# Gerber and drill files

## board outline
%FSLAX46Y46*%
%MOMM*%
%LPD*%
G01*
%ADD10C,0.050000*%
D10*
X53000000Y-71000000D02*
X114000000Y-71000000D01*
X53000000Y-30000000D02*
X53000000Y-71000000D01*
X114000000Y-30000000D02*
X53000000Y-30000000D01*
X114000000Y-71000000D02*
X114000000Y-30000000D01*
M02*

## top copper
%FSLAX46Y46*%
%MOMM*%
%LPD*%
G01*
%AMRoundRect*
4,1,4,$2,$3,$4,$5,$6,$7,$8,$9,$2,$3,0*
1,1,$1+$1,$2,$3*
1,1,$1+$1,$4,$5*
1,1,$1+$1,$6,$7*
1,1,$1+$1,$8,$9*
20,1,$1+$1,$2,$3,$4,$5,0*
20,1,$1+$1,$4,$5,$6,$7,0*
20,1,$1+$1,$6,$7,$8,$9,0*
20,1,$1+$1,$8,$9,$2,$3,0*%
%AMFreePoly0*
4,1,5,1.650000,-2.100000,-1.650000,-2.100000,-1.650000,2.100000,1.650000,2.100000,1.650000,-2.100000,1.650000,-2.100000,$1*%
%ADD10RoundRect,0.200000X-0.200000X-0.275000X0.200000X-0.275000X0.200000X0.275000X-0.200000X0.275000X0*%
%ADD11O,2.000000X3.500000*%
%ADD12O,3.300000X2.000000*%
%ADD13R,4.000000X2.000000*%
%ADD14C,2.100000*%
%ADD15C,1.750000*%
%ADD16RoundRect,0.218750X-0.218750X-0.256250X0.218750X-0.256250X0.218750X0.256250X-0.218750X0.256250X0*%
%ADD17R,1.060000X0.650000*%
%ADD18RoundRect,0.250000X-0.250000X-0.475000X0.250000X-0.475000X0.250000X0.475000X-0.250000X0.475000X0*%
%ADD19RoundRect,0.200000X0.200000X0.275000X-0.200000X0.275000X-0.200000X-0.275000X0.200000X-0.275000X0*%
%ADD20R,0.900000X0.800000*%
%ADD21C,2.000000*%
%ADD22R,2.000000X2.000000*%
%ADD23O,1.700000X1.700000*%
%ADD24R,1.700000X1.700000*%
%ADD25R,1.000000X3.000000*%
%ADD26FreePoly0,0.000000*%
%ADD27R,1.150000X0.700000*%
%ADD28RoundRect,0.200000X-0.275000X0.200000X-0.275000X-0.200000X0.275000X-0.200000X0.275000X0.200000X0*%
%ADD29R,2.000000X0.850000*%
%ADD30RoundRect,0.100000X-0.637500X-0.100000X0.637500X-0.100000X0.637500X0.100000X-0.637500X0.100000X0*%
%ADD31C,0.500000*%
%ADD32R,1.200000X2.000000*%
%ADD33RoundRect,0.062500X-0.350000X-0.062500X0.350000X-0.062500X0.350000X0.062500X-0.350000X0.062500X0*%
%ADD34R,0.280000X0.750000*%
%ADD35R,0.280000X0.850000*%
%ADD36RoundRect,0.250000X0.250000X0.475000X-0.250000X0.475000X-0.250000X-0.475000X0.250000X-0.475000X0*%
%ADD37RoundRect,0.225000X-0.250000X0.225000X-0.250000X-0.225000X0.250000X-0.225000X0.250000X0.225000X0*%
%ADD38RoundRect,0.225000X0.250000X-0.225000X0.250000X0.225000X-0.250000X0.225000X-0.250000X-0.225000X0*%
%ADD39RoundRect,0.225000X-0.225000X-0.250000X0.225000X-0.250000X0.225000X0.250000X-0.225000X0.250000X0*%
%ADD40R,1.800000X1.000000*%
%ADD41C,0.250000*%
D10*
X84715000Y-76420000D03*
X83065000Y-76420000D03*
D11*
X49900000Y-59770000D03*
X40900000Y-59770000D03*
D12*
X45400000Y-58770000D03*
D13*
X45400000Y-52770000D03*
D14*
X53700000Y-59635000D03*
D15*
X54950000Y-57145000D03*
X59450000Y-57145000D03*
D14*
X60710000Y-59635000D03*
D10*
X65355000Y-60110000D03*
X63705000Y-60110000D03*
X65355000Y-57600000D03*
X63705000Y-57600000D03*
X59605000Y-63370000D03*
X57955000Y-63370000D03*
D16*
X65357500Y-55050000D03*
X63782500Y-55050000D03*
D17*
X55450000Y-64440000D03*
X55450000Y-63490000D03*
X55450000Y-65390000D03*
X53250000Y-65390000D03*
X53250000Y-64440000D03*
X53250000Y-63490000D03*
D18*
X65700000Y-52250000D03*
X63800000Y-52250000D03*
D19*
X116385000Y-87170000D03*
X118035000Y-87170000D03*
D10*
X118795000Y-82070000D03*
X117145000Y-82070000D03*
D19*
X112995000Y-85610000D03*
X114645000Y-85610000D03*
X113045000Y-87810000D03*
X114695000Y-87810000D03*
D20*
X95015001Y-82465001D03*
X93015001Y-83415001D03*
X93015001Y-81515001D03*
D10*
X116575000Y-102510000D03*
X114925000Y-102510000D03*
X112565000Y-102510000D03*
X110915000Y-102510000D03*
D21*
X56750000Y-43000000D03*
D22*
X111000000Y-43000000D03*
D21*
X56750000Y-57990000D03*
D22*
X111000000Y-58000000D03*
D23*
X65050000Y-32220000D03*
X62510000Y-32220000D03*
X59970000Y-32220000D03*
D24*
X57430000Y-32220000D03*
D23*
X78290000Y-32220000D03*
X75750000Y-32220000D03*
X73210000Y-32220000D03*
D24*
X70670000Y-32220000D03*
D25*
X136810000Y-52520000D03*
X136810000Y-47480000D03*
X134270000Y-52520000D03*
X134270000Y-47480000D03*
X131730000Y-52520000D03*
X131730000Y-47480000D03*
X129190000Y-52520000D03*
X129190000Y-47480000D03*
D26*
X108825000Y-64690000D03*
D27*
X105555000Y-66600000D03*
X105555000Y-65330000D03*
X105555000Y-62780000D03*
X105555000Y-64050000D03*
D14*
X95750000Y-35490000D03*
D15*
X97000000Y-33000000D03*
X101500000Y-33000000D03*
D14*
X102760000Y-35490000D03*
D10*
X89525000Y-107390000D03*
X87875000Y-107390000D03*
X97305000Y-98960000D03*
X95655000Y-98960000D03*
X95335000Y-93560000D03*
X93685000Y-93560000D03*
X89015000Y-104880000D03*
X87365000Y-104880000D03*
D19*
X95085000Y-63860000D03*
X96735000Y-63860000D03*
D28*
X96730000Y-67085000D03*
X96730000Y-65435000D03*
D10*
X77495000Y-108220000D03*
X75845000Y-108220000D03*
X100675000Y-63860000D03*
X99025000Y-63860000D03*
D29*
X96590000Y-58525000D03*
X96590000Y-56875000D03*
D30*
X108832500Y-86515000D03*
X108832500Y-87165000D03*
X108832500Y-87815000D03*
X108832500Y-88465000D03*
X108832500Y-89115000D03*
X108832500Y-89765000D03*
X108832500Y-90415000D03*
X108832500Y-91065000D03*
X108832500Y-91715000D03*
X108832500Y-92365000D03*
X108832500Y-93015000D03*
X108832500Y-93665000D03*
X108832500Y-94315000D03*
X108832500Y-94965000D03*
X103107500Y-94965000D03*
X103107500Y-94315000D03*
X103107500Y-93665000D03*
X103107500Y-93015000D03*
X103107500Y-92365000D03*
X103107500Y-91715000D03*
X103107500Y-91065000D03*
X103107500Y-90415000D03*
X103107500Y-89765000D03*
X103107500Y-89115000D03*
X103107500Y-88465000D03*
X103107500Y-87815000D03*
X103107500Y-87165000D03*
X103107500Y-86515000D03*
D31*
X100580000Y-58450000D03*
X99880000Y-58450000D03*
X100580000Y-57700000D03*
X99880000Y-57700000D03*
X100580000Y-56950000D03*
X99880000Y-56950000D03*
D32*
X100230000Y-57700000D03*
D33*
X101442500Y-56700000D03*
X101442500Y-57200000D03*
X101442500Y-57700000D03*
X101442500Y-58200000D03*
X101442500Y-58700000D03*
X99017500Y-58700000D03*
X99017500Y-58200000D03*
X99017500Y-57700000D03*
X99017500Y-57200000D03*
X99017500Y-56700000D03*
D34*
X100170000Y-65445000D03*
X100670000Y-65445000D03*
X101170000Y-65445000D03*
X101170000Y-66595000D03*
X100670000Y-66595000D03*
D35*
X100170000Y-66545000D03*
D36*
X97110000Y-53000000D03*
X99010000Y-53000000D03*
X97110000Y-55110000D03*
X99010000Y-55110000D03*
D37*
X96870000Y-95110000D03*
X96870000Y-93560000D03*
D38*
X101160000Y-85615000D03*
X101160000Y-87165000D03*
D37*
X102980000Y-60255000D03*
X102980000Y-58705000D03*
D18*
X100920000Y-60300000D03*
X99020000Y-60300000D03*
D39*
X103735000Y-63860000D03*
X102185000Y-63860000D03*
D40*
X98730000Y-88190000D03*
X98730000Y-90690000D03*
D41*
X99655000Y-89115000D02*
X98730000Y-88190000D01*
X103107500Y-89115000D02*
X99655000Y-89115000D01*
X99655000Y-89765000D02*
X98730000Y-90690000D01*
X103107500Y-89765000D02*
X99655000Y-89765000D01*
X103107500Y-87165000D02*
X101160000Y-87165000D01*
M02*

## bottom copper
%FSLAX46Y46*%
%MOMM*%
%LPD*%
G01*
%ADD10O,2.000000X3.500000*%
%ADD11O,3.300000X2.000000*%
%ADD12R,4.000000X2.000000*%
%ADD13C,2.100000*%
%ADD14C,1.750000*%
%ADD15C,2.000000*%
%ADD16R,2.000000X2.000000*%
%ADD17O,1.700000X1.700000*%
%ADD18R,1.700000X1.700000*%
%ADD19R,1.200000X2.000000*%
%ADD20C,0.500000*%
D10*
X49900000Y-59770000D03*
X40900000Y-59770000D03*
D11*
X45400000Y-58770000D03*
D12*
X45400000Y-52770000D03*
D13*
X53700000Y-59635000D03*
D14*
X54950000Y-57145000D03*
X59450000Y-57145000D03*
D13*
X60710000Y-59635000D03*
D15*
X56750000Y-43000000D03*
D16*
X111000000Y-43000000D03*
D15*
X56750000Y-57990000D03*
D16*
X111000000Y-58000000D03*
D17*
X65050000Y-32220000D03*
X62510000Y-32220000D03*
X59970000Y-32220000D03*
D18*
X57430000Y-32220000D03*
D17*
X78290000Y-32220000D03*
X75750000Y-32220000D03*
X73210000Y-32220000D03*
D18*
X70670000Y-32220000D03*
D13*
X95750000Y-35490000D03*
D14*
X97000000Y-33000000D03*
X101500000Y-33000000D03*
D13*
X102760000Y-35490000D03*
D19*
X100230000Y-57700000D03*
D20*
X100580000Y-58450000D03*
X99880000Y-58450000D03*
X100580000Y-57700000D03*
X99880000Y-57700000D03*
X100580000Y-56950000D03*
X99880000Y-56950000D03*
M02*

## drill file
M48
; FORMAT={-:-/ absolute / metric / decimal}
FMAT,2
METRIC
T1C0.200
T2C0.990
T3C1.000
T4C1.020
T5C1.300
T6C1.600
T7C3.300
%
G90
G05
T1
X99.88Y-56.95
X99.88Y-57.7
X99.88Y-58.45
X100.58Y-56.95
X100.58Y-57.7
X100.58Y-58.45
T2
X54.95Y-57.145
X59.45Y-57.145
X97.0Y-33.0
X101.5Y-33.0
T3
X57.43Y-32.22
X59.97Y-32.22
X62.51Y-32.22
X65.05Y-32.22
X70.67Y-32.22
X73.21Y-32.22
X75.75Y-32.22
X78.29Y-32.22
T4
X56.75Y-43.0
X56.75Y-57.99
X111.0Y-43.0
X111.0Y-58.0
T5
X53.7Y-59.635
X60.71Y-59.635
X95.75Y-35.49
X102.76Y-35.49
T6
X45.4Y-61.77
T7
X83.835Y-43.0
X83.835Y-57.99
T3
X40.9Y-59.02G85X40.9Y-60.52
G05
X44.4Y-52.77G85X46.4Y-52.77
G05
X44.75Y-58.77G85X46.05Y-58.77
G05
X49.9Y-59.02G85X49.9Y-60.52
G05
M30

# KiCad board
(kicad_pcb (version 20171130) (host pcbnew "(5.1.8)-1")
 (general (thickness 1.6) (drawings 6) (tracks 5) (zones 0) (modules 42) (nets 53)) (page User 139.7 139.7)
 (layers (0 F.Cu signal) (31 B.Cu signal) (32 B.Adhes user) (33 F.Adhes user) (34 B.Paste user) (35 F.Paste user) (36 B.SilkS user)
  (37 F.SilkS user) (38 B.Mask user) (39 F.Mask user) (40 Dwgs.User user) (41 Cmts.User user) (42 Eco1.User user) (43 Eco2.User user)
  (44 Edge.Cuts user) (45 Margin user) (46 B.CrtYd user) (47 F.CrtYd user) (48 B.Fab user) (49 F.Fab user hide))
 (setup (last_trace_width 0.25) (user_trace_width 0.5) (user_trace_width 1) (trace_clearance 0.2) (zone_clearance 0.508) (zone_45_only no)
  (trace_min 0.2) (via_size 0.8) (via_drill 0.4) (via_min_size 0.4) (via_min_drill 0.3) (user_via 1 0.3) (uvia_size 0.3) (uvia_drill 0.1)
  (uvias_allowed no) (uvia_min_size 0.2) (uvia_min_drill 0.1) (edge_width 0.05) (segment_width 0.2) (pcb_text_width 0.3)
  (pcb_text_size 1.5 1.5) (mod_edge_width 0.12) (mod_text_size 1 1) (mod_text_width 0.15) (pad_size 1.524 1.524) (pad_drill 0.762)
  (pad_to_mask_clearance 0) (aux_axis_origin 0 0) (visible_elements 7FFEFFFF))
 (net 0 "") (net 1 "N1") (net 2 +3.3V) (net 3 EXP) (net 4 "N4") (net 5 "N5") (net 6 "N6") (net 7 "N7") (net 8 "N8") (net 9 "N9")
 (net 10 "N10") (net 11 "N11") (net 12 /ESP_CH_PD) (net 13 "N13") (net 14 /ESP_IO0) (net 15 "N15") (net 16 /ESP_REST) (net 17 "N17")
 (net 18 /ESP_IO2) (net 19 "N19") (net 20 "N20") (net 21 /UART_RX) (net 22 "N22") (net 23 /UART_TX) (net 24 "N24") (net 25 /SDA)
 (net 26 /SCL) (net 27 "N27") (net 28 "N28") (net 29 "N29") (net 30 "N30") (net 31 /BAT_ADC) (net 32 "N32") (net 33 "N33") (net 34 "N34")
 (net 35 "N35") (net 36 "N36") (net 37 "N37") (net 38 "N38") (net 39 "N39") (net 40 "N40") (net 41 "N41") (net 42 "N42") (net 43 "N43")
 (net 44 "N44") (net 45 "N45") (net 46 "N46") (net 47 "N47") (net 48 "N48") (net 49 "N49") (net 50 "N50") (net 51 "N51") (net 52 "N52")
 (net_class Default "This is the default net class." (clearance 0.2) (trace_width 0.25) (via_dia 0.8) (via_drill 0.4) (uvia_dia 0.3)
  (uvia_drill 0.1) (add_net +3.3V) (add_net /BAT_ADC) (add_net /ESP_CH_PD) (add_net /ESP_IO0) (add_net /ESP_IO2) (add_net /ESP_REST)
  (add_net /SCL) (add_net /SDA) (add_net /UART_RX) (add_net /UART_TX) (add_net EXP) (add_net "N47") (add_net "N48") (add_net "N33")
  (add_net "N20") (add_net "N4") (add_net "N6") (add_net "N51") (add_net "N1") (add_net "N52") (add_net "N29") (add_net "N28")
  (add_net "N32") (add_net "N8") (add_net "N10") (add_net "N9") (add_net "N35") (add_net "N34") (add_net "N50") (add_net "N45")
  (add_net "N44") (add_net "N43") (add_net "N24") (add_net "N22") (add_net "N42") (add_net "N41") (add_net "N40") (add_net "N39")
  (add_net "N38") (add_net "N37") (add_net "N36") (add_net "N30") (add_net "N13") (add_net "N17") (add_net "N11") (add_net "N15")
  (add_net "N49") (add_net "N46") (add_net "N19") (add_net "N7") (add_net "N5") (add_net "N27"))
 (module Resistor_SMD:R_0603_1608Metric (layer F.Cu) (at 83.89 76.42)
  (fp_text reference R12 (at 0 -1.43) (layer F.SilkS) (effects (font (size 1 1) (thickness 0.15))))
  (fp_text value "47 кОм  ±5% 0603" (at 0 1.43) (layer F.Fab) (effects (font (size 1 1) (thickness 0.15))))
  (pad 2 smd roundrect (at 0.825 0) (size 0.8 0.95) (layers F.Cu F.Paste F.Mask) (roundrect_rratio 0.25) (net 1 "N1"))
  (pad 1 smd roundrect (at -0.825 0) (size 0.8 0.95) (layers F.Cu F.Paste F.Mask) (roundrect_rratio 0.25) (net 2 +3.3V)))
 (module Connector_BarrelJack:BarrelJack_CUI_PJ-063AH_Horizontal (layer F.Cu) (at 45.4 52.77)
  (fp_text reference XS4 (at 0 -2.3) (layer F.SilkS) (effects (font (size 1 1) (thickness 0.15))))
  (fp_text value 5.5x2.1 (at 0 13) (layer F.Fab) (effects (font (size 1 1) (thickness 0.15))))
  (pad "" np_thru_hole circle (at 0 9) (size 1.6 1.6) (drill 1.6) (layers *.Cu *.Mask))
  (pad MP thru_hole oval (at 4.5 7) (size 2 3.5) (drill oval 1 2.5) (layers *.Cu *.Mask))
  (pad MP thru_hole oval (at -4.5 7) (size 2 3.5) (drill oval 1 2.5) (layers *.Cu *.Mask))
  (pad 2 thru_hole oval (at 0 6) (size 3.3 2) (drill oval 2.3 1) (layers *.Cu *.Mask) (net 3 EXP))
  (pad 1 thru_hole rect (at 0 0) (size 4 2) (drill oval 3 1) (layers *.Cu *.Mask) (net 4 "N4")))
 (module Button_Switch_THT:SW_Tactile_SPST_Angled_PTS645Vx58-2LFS (layer F.Cu) (at 54.95 57.145)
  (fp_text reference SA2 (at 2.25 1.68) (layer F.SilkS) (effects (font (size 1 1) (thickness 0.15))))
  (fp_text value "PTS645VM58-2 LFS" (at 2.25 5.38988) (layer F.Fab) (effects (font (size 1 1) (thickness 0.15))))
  (pad "" thru_hole circle (at -1.25 2.49) (size 2.1 2.1) (drill 1.3) (layers *.Cu *.Mask))
  (pad 1 thru_hole circle (at 0 0) (size 1.75 1.75) (drill 0.99) (layers *.Cu *.Mask) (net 1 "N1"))
  (pad 2 thru_hole circle (at 4.5 0) (size 1.75 1.75) (drill 0.99) (layers *.Cu *.Mask) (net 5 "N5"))
  (pad "" thru_hole circle (at 5.76 2.49) (size 2.1 2.1) (drill 1.3) (layers *.Cu *.Mask)))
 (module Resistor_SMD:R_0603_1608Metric (layer F.Cu) (at 64.53 60.11)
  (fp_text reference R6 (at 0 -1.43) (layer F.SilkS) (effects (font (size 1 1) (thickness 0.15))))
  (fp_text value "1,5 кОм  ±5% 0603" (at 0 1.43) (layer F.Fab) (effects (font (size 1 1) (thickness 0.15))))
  (pad 2 smd roundrect (at 0.825 0) (size 0.8 0.95) (layers F.Cu F.Paste F.Mask) (roundrect_rratio 0.25) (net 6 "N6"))
  (pad 1 smd roundrect (at -0.825 0) (size 0.8 0.95) (layers F.Cu F.Paste F.Mask) (roundrect_rratio 0.25) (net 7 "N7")))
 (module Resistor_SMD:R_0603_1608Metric (layer F.Cu) (at 64.53 57.6)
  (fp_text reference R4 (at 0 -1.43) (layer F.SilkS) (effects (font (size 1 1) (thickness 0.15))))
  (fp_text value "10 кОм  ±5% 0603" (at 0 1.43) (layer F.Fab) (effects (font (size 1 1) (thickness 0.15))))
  (pad 2 smd roundrect (at 0.825 0) (size 0.8 0.95) (layers F.Cu F.Paste F.Mask) (roundrect_rratio 0.25) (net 3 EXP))
  (pad 1 smd roundrect (at -0.825 0) (size 0.8 0.95) (layers F.Cu F.Paste F.Mask) (roundrect_rratio 0.25) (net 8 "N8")))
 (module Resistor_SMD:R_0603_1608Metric (layer F.Cu) (at 58.78 63.37)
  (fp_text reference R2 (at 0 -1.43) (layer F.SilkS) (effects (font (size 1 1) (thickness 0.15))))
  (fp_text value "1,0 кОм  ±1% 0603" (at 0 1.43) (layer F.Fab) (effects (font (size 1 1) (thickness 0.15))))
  (pad 2 smd roundrect (at 0.825 0) (size 0.8 0.95) (layers F.Cu F.Paste F.Mask) (roundrect_rratio 0.25) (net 3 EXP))
  (pad 1 smd roundrect (at -0.825 0) (size 0.8 0.95) (layers F.Cu F.Paste F.Mask) (roundrect_rratio 0.25) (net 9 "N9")))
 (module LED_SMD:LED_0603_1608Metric (layer F.Cu) (at 64.57 55.05)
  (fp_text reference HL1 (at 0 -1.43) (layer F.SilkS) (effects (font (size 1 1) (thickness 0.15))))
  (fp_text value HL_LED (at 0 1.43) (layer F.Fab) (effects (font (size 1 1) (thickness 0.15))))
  (pad 2 smd roundrect (at 0.7875 0) (size 0.875 0.95) (layers F.Cu F.Paste F.Mask) (roundrect_rratio 0.25) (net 7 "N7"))
  (pad 1 smd roundrect (at -0.7875 0) (size 0.875 0.95) (layers F.Cu F.Paste F.Mask) (roundrect_rratio 0.25) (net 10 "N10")))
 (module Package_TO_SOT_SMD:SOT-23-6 (layer F.Cu) (at 54.35 64.44)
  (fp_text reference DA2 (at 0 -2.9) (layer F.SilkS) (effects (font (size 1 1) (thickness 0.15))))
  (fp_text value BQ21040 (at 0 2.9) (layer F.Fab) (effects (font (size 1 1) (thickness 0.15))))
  (pad 5 smd rect (at 1.1 0) (size 1.06 0.65) (layers F.Cu F.Paste F.Mask) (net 3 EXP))
  (pad 6 smd rect (at 1.1 -0.95) (size 1.06 0.65) (layers F.Cu F.Paste F.Mask) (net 4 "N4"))
  (pad 4 smd rect (at 1.1 0.95) (size 1.06 0.65) (layers F.Cu F.Paste F.Mask) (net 9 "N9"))
  (pad 3 smd rect (at -1.1 0.95) (size 1.06 0.65) (layers F.Cu F.Paste F.Mask) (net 10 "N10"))
  (pad 2 smd rect (at -1.1 0) (size 1.06 0.65) (layers F.Cu F.Paste F.Mask) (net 6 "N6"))
  (pad 1 smd rect (at -1.1 -0.95) (size 1.06 0.65) (layers F.Cu F.Paste F.Mask) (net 8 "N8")))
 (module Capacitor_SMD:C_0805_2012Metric (layer F.Cu) (at 64.75 52.25)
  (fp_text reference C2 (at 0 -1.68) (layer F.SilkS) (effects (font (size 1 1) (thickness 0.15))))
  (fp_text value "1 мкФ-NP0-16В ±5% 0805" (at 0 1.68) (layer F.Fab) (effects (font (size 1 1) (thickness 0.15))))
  (pad 2 smd roundrect (at 0.95 0) (size 1 1.45) (layers F.Cu F.Paste F.Mask) (roundrect_rratio 0.25) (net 3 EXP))
  (pad 1 smd roundrect (at -0.95 0) (size 1 1.45) (layers F.Cu F.Paste F.Mask) (roundrect_rratio 0.25) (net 4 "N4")))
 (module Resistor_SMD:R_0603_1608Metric (layer F.Cu) (at 117.21 87.17 180)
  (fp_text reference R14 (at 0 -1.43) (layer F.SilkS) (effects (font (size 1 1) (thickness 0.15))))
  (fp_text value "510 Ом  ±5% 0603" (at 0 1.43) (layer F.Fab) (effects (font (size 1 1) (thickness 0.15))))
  (pad 2 smd roundrect (at 0.825 0 180) (size 0.8 0.95) (layers F.Cu F.Paste F.Mask) (roundrect_rratio 0.25) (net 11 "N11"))
  (pad 1 smd roundrect (at -0.825 0 180) (size 0.8 0.95) (layers F.Cu F.Paste F.Mask) (roundrect_rratio 0.25) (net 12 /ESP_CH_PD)))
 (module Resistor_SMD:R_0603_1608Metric (layer F.Cu) (at 117.97 82.07)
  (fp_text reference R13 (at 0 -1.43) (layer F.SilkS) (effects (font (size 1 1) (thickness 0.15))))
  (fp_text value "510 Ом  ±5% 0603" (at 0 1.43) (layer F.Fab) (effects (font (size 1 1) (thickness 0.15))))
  (pad 2 smd roundrect (at 0.825 0) (size 0.8 0.95) (layers F.Cu F.Paste F.Mask) (roundrect_rratio 0.25) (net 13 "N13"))
  (pad 1 smd roundrect (at -0.825 0) (size 0.8 0.95) (layers F.Cu F.Paste F.Mask) (roundrect_rratio 0.25) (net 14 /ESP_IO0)))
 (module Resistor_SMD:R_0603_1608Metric (layer F.Cu) (at 113.82 85.61 180)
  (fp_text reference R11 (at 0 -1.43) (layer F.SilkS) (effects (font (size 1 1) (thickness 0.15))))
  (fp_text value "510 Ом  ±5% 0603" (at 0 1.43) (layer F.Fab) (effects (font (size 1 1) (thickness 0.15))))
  (pad 2 smd roundrect (at 0.825 0 180) (size 0.8 0.95) (layers F.Cu F.Paste F.Mask) (roundrect_rratio 0.25) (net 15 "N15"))
  (pad 1 smd roundrect (at -0.825 0 180) (size 0.8 0.95) (layers F.Cu F.Paste F.Mask) (roundrect_rratio 0.25) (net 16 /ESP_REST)))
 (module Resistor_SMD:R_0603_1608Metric (layer F.Cu) (at 113.87 87.81 180)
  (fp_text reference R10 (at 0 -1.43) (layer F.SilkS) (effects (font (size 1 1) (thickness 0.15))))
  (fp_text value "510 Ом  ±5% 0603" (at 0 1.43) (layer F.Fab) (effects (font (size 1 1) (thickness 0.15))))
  (pad 2 smd roundrect (at 0.825 0 180) (size 0.8 0.95) (layers F.Cu F.Paste F.Mask) (roundrect_rratio 0.25) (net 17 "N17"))
  (pad 1 smd roundrect (at -0.825 0 180) (size 0.8 0.95) (layers F.Cu F.Paste F.Mask) (roundrect_rratio 0.25) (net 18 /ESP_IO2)))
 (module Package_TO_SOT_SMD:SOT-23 (layer F.Cu) (at 94.015001 82.465001)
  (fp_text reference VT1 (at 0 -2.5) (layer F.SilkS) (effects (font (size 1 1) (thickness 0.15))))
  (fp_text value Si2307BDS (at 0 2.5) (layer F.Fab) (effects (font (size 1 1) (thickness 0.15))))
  (pad 3 smd rect (at 1 0) (size 0.9 0.8) (layers F.Cu F.Paste F.Mask) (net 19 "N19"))
  (pad 2 smd rect (at -1 0.95) (size 0.9 0.8) (layers F.Cu F.Paste F.Mask) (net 6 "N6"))
  (pad 1 smd rect (at -1 -0.95) (size 0.9 0.8) (layers F.Cu F.Paste F.Mask) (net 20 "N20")))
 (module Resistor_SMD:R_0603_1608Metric (layer F.Cu) (at 115.75 102.51)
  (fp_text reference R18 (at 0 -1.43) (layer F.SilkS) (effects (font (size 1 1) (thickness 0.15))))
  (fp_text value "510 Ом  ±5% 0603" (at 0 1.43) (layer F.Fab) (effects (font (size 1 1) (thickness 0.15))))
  (pad 2 smd roundrect (at 0.825 0) (size 0.8 0.95) (layers F.Cu F.Paste F.Mask) (roundrect_rratio 0.25) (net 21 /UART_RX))
  (pad 1 smd roundrect (at -0.825 0) (size 0.8 0.95) (layers F.Cu F.Paste F.Mask) (roundrect_rratio 0.25) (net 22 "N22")))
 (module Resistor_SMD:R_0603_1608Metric (layer F.Cu) (at 111.74 102.51)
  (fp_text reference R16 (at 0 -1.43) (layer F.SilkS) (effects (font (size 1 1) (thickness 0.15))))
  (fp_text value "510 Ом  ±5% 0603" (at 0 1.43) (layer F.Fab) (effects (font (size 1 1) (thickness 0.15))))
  (pad 2 smd roundrect (at 0.825 0) (size 0.8 0.95) (layers F.Cu F.Paste F.Mask) (roundrect_rratio 0.25) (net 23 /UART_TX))
  (pad 1 smd roundrect (at -0.825 0) (size 0.8 0.95) (layers F.Cu F.Paste F.Mask) (roundrect_rratio 0.25) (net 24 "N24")))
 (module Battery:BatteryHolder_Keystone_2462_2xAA (layer B.Cu) (at 111 43 180)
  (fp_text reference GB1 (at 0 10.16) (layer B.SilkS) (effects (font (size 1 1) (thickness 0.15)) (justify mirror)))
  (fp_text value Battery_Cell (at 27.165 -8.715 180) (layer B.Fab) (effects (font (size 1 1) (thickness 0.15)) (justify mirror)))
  (pad "" np_thru_hole circle (at 27.165 0 180) (size 3.3 3.3) (drill 3.3) (layers *.Cu *.Mask))
  (pad "" np_thru_hole circle (at 27.165 -14.99 180) (size 3.3 3.3) (drill 3.3) (layers *.Cu *.Mask))
  (pad 2 thru_hole circle (at 54.25 0 180) (size 2 2) (drill 1.02) (layers *.Cu *.Mask) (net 20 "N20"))
  (pad 1 thru_hole rect (at 0 0 180) (size 2 2) (drill 1.02) (layers *.Cu *.Mask) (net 19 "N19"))
  (pad 2 thru_hole circle (at 54.25 -14.99 180) (size 2 2) (drill 1.02) (layers *.Cu *.Mask) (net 20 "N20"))
  (pad 1 thru_hole rect (at 0 -15 180) (size 2 2) (drill 1.02) (layers *.Cu *.Mask) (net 19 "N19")))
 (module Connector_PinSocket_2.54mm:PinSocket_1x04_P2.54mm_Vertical (layer F.Cu) (at 57.43 32.22 90)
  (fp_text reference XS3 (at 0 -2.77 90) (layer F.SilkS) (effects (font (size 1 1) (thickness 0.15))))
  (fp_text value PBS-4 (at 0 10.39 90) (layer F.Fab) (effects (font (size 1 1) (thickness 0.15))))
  (pad 4 thru_hole oval (at 0 7.62 90) (size 1.7 1.7) (drill 1) (layers *.Cu *.Mask) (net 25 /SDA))
  (pad 3 thru_hole oval (at 0 5.08 90) (size 1.7 1.7) (drill 1) (layers *.Cu *.Mask) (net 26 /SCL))
  (pad 2 thru_hole oval (at 0 2.54 90) (size 1.7 1.7) (drill 1) (layers *.Cu *.Mask) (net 2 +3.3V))
  (pad 1 thru_hole rect (at 0 0 90) (size 1.7 1.7) (drill 1) (layers *.Cu *.Mask) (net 3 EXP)))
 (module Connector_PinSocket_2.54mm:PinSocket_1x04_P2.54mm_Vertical (layer F.Cu) (at 70.67 32.22 90)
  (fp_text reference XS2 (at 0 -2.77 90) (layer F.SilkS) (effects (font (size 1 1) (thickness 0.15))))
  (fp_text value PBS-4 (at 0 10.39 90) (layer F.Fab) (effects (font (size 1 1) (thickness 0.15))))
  (pad 4 thru_hole oval (at 0 7.62 90) (size 1.7 1.7) (drill 1) (layers *.Cu *.Mask) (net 25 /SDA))
  (pad 3 thru_hole oval (at 0 5.08 90) (size 1.7 1.7) (drill 1) (layers *.Cu *.Mask) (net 26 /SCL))
  (pad 2 thru_hole oval (at 0 2.54 90) (size 1.7 1.7) (drill 1) (layers *.Cu *.Mask) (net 3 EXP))
  (pad 1 thru_hole rect (at 0 0 90) (size 1.7 1.7) (drill 1) (layers *.Cu *.Mask) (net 2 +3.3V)))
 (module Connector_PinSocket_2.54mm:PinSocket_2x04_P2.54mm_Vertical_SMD (layer F.Cu) (at 133 50 90)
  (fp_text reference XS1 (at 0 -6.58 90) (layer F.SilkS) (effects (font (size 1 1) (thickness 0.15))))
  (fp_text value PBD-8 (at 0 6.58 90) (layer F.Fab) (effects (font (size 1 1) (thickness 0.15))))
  (pad 8 smd rect (at -2.52 3.81 90) (size 3 1) (layers F.Cu F.Paste F.Mask) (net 21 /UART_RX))
  (pad 7 smd rect (at 2.52 3.81 90) (size 3 1) (layers F.Cu F.Paste F.Mask) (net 16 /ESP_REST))
  (pad 6 smd rect (at -2.52 1.27 90) (size 3 1) (layers F.Cu F.Paste F.Mask) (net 12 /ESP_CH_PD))
  (pad 5 smd rect (at 2.52 1.27 90) (size 3 1) (layers F.Cu F.Paste F.Mask) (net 2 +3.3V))
  (pad 4 smd rect (at -2.52 -1.27 90) (size 3 1) (layers F.Cu F.Paste F.Mask) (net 23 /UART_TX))
  (pad 3 smd rect (at 2.52 -1.27 90) (size 3 1) (layers F.Cu F.Paste F.Mask) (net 14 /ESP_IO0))
  (pad 2 smd rect (at -2.52 -3.81 90) (size 3 1) (layers F.Cu F.Paste F.Mask) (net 18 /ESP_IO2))
  (pad 1 smd rect (at 2.52 -3.81 90) (size 3 1) (layers F.Cu F.Paste F.Mask) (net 3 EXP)))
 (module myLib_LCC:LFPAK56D (layer F.Cu) (at 108.39 64.69) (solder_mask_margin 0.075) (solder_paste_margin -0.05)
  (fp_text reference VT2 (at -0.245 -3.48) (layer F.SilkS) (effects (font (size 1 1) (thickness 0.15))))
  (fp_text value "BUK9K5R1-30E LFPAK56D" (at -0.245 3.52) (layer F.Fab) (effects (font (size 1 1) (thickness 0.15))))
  (pad 5 smd custom (at 0.435 0) (size 3.3 4.2) (layers F.Cu F.Mask) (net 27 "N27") (solder_mask_margin 0.07) (zone_connect 2)
   (options (clearance outline) (anchor rect)) (primitives))
  (pad "" smd rect (at 0.185 0) (size 0.6 0.9) (layers F.Paste))
  (pad 6 smd rect (at 2.885 0.6 270) (size 0.6 0.9) (layers F.Paste) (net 27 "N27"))
  (pad 4 smd rect (at -2.835 1.91 270) (size 0.7 1.15) (layers F.Cu F.Paste F.Mask) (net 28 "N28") (solder_mask_margin 0.07)
   (solder_paste_margin -0.05))
  (pad 3 smd rect (at -2.835 0.64 270) (size 0.7 1.15) (layers F.Cu F.Paste F.Mask) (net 20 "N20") (solder_mask_margin 0.07)
   (solder_paste_margin -0.05))
  (pad 1 smd rect (at -2.835 -1.91 270) (size 0.7 1.15) (layers F.Cu F.Paste F.Mask) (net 3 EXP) (solder_mask_margin 0.07)
   (solder_paste_margin -0.05))
  (pad 2 smd rect (at -2.835 -0.64 270) (size 0.7 1.15) (layers F.Cu F.Paste F.Mask) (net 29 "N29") (solder_mask_margin 0.07)
   (solder_paste_margin -0.05))
  (pad "" smd rect (at 2.885 -0.6 270) (size 0.6 0.9) (layers F.Paste))
  (pad 7 smd rect (at 2.885 1.88 270) (size 0.6 0.9) (layers F.Paste) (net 27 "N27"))
  (pad "" smd rect (at 2.885 -1.88 270) (size 0.6 0.9) (layers F.Paste))
  (pad "" smd rect (at -0.665 0) (size 0.6 0.9) (layers F.Paste))
  (pad "" smd rect (at 1.035 0) (size 0.6 0.9) (layers F.Paste))
  (pad "" smd rect (at 1.035 1.15) (size 0.6 0.9) (layers F.Paste))
  (pad "" smd rect (at -0.665 1.15) (size 0.6 0.9) (layers F.Paste))
  (pad 8 smd rect (at 0.185 1.15) (size 0.6 0.9) (layers F.Paste) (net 27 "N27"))
  (pad "" smd rect (at 1.035 -1.15) (size 0.6 0.9) (layers F.Paste))
  (pad "" smd rect (at -0.665 -1.15) (size 0.6 0.9) (layers F.Paste))
  (pad "" smd rect (at 0.185 -1.15) (size 0.6 0.9) (layers F.Paste)))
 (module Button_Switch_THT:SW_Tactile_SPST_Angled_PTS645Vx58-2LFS (layer F.Cu) (at 97 33)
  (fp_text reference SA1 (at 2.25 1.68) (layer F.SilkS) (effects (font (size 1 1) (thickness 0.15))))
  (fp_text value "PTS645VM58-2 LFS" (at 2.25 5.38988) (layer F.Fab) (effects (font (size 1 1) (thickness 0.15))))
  (pad "" thru_hole circle (at -1.25 2.49) (size 2.1 2.1) (drill 1.3) (layers *.Cu *.Mask))
  (pad 1 thru_hole circle (at 0 0) (size 1.75 1.75) (drill 0.99) (layers *.Cu *.Mask) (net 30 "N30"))
  (pad 2 thru_hole circle (at 4.5 0) (size 1.75 1.75) (drill 0.99) (layers *.Cu *.Mask) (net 2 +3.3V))
  (pad "" thru_hole circle (at 5.76 2.49) (size 2.1 2.1) (drill 1.3) (layers *.Cu *.Mask)))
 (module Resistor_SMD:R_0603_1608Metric (layer F.Cu) (at 88.7 107.39)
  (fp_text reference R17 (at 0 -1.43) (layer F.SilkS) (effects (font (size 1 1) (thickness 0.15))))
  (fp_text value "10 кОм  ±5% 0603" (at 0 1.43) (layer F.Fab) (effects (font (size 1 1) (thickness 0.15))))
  (pad 2 smd roundrect (at 0.825 0) (size 0.8 0.95) (layers F.Cu F.Paste F.Mask) (roundrect_rratio 0.25) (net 26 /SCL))
  (pad 1 smd roundrect (at -0.825 0) (size 0.8 0.95) (layers F.Cu F.Paste F.Mask) (roundrect_rratio 0.25) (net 2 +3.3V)))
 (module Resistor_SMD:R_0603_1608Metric (layer F.Cu) (at 96.48 98.96)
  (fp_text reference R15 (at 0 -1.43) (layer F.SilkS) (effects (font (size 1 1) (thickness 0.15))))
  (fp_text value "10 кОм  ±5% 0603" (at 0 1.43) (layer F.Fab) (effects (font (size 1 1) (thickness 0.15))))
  (pad 2 smd roundrect (at 0.825 0) (size 0.8 0.95) (layers F.Cu F.Paste F.Mask) (roundrect_rratio 0.25) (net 25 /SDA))
  (pad 1 smd roundrect (at -0.825 0) (size 0.8 0.95) (layers F.Cu F.Paste F.Mask) (roundrect_rratio 0.25) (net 2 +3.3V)))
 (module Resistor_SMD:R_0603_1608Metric (layer F.Cu) (at 94.51 93.56)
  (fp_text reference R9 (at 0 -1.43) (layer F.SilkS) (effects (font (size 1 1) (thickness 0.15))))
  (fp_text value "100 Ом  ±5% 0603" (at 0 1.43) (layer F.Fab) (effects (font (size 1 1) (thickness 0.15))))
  (pad 2 smd roundrect (at 0.825 0) (size 0.8 0.95) (layers F.Cu F.Paste F.Mask) (roundrect_rratio 0.25) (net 5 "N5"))
  (pad 1 smd roundrect (at -0.825 0) (size 0.8 0.95) (layers F.Cu F.Paste F.Mask) (roundrect_rratio 0.25) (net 3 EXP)))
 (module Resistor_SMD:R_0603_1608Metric (layer F.Cu) (at 88.19 104.88)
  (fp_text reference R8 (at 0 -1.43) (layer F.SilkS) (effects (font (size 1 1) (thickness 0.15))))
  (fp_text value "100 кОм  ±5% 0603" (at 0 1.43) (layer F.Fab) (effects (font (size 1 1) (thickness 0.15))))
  (pad 2 smd roundrect (at 0.825 0) (size 0.8 0.95) (layers F.Cu F.Paste F.Mask) (roundrect_rratio 0.25) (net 3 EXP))
  (pad 1 smd roundrect (at -0.825 0) (size 0.8 0.95) (layers F.Cu F.Paste F.Mask) (roundrect_rratio 0.25) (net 30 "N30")))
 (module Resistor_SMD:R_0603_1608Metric (layer F.Cu) (at 95.91 63.86 180)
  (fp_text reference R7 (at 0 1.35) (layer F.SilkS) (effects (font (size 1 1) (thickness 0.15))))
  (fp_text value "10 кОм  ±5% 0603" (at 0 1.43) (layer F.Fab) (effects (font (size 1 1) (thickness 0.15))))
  (pad 2 smd roundrect (at 0.825 0 180) (size 0.8 0.95) (layers F.Cu F.Paste F.Mask) (roundrect_rratio 0.25) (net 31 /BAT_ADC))
  (pad 1 smd roundrect (at -0.825 0 180) (size 0.8 0.95) (layers F.Cu F.Paste F.Mask) (roundrect_rratio 0.25) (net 6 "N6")))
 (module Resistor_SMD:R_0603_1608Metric (layer F.Cu) (at 96.73 66.26 270)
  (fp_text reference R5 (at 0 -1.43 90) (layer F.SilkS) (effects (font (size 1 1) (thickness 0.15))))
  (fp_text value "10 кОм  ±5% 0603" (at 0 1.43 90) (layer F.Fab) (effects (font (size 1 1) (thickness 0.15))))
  (pad 2 smd roundrect (at 0.825 0 270) (size 0.8 0.95) (layers F.Cu F.Paste F.Mask) (roundrect_rratio 0.25) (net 3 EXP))
  (pad 1 smd roundrect (at -0.825 0 270) (size 0.8 0.95) (layers F.Cu F.Paste F.Mask) (roundrect_rratio 0.25) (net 6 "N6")))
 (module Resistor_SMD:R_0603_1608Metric (layer F.Cu) (at 76.67 108.22)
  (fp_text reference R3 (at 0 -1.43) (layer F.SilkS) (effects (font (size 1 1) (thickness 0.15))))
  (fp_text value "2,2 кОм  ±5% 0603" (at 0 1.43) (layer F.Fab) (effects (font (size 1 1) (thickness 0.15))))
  (pad 2 smd roundrect (at 0.825 0) (size 0.8 0.95) (layers F.Cu F.Paste F.Mask) (roundrect_rratio 0.25) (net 3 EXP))
  (pad 1 smd roundrect (at -0.825 0) (size 0.8 0.95) (layers F.Cu F.Paste F.Mask) (roundrect_rratio 0.25) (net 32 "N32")))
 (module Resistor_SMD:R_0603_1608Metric (layer F.Cu) (at 99.85 63.86)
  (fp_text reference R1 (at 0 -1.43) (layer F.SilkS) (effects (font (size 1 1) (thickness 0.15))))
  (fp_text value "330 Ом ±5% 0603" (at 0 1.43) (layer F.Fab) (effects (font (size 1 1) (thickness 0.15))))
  (pad 2 smd roundrect (at 0.825 0) (size 0.8 0.95) (layers F.Cu F.Paste F.Mask) (roundrect_rratio 0.25) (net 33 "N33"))
  (pad 1 smd roundrect (at -0.825 0) (size 0.8 0.95) (layers F.Cu F.Paste F.Mask) (roundrect_rratio 0.25) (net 6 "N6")))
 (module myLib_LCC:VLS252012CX (layer F.Cu) (at 97.59 58.95 90)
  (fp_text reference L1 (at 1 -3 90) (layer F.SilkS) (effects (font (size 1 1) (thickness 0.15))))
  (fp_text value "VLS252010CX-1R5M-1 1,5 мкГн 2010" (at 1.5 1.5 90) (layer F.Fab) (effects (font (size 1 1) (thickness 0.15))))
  (pad 1 smd rect (at 0.425 -1 90) (size 0.85 2) (layers F.Cu F.Paste F.Mask) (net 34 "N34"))
  (pad 2 smd rect (at 2.075 -1 90) (size 0.85 2) (layers F.Cu F.Paste F.Mask) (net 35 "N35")))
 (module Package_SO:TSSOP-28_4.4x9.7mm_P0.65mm (layer F.Cu) (at 105.97 90.74)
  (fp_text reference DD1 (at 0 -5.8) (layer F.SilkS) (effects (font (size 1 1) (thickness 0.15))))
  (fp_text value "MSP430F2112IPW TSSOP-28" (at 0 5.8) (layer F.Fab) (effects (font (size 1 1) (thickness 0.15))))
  (pad 28 smd roundrect (at 2.8625 -4.225) (size 1.475 0.4) (layers F.Cu F.Paste F.Mask) (roundrect_rratio 0.25) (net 15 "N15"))
  (pad 27 smd roundrect (at 2.8625 -3.575) (size 1.475 0.4) (layers F.Cu F.Paste F.Mask) (roundrect_rratio 0.25) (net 11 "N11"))
  (pad 26 smd roundrect (at 2.8625 -2.925) (size 1.475 0.4) (layers F.Cu F.Paste F.Mask) (roundrect_rratio 0.25) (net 17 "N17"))
  (pad 25 smd roundrect (at 2.8625 -2.275) (size 1.475 0.4) (layers F.Cu F.Paste F.Mask) (roundrect_rratio 0.25) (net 13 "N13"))
  (pad 24 smd roundrect (at 2.8625 -1.625) (size 1.475 0.4) (layers F.Cu F.Paste F.Mask) (roundrect_rratio 0.25) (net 30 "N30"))
  (pad 23 smd roundrect (at 2.8625 -0.975) (size 1.475 0.4) (layers F.Cu F.Paste F.Mask) (roundrect_rratio 0.25) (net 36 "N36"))
  (pad 22 smd roundrect (at 2.8625 -0.325) (size 1.475 0.4) (layers F.Cu F.Paste F.Mask) (roundrect_rratio 0.25) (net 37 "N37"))
  (pad 21 smd roundrect (at 2.8625 0.325) (size 1.475 0.4) (layers F.Cu F.Paste F.Mask) (roundrect_rratio 0.25) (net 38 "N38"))
  (pad 20 smd roundrect (at 2.8625 0.975) (size 1.475 0.4) (layers F.Cu F.Paste F.Mask) (roundrect_rratio 0.25) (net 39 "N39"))
  (pad 19 smd roundrect (at 2.8625 1.625) (size 1.475 0.4) (layers F.Cu F.Paste F.Mask) (roundrect_rratio 0.25) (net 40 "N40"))
  (pad 18 smd roundrect (at 2.8625 2.275) (size 1.475 0.4) (layers F.Cu F.Paste F.Mask) (roundrect_rratio 0.25) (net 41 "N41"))
  (pad 17 smd roundrect (at 2.8625 2.925) (size 1.475 0.4) (layers F.Cu F.Paste F.Mask) (roundrect_rratio 0.25) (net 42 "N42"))
  (pad 16 smd roundrect (at 2.8625 3.575) (size 1.475 0.4) (layers F.Cu F.Paste F.Mask) (roundrect_rratio 0.25) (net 22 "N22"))
  (pad 15 smd roundrect (at 2.8625 4.225) (size 1.475 0.4) (layers F.Cu F.Paste F.Mask) (roundrect_rratio 0.25) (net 24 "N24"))
  (pad 14 smd roundrect (at -2.8625 4.225) (size 1.475 0.4) (layers F.Cu F.Paste F.Mask) (roundrect_rratio 0.25) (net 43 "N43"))
  (pad 13 smd roundrect (at -2.8625 3.575) (size 1.475 0.4) (layers F.Cu F.Paste F.Mask) (roundrect_rratio 0.25) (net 26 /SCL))
  (pad 12 smd roundrect (at -2.8625 2.925) (size 1.475 0.4) (layers F.Cu F.Paste F.Mask) (roundrect_rratio 0.25) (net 25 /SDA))
  (pad 11 smd roundrect (at -2.8625 2.275) (size 1.475 0.4) (layers F.Cu F.Paste F.Mask) (roundrect_rratio 0.25) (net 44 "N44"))
  (pad 10 smd roundrect (at -2.8625 1.625) (size 1.475 0.4) (layers F.Cu F.Paste F.Mask) (roundrect_rratio 0.25) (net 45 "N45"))
  (pad 9 smd roundrect (at -2.8625 0.975) (size 1.475 0.4) (layers F.Cu F.Paste F.Mask) (roundrect_rratio 0.25) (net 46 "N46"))
  (pad 8 smd roundrect (at -2.8625 0.325) (size 1.475 0.4) (layers F.Cu F.Paste F.Mask) (roundrect_rratio 0.25) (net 31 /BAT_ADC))
  (pad 7 smd roundrect (at -2.8625 -0.325) (size 1.475 0.4) (layers F.Cu F.Paste F.Mask) (roundrect_rratio 0.25) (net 1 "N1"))
  (pad 6 smd roundrect (at -2.8625 -0.975) (size 1.475 0.4) (layers F.Cu F.Paste F.Mask) (roundrect_rratio 0.25) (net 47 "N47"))
  (pad 5 smd roundrect (at -2.8625 -1.625) (size 1.475 0.4) (layers F.Cu F.Paste F.Mask) (roundrect_rratio 0.25) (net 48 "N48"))
  (pad 4 smd roundrect (at -2.8625 -2.275) (size 1.475 0.4) (layers F.Cu F.Paste F.Mask) (roundrect_rratio 0.25) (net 3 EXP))
  (pad 3 smd roundrect (at -2.8625 -2.925) (size 1.475 0.4) (layers F.Cu F.Paste F.Mask) (roundrect_rratio 0.25) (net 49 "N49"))
  (pad 2 smd roundrect (at -2.8625 -3.575) (size 1.475 0.4) (layers F.Cu F.Paste F.Mask) (roundrect_rratio 0.25) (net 2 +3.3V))
  (pad 1 smd roundrect (at -2.8625 -4.225) (size 1.475 0.4) (layers F.Cu F.Paste F.Mask) (roundrect_rratio 0.25) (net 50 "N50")))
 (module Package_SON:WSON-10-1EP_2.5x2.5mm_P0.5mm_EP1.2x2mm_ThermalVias (layer F.Cu) (at 100.23 57.7)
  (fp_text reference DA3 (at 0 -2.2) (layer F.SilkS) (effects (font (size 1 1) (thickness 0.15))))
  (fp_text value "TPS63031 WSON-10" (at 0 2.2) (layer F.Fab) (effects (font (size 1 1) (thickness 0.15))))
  (pad "" smd roundrect (at 0.3 0.5) (size 0.52 0.87) (layers F.Paste) (roundrect_rratio 0.25))
  (pad "" smd roundrect (at 0.3 -0.5) (size 0.52 0.87) (layers F.Paste) (roundrect_rratio 0.25))
  (pad "" smd roundrect (at -0.3 0.5) (size 0.52 0.87) (layers F.Paste) (roundrect_rratio 0.25))
  (pad "" smd roundrect (at -0.3 -0.5) (size 0.52 0.87) (layers F.Paste) (roundrect_rratio 0.25))
  (pad 11 smd rect (at 0 0) (size 1.2 2) (layers B.Cu) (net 3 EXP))
  (pad 11 thru_hole circle (at 0.35 0.75) (size 0.5 0.5) (drill 0.2) (layers *.Cu) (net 3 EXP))
  (pad 11 thru_hole circle (at -0.35 0.75) (size 0.5 0.5) (drill 0.2) (layers *.Cu) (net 3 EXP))
  (pad 11 thru_hole circle (at 0.35 0) (size 0.5 0.5) (drill 0.2) (layers *.Cu) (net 3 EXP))
  (pad 11 thru_hole circle (at -0.35 0) (size 0.5 0.5) (drill 0.2) (layers *.Cu) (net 3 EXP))
  (pad 11 thru_hole circle (at 0.35 -0.75) (size 0.5 0.5) (drill 0.2) (layers *.Cu) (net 3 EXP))
  (pad 11 thru_hole circle (at -0.35 -0.75) (size 0.5 0.5) (drill 0.2) (layers *.Cu) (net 3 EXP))
  (pad 11 smd rect (at 0 0) (size 1.2 2) (layers F.Cu F.Mask) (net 3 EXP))
  (pad 10 smd roundrect (at 1.2125 -1) (size 0.825 0.25) (layers F.Cu F.Paste F.Mask) (roundrect_rratio 0.25) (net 2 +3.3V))
  (pad 9 smd roundrect (at 1.2125 -0.5) (size 0.825 0.25) (layers F.Cu F.Paste F.Mask) (roundrect_rratio 0.25) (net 3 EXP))
  (pad 8 smd roundrect (at 1.2125 0) (size 0.825 0.25) (layers F.Cu F.Paste F.Mask) (roundrect_rratio 0.25) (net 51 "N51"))
  (pad 7 smd roundrect (at 1.2125 0.5) (size 0.825 0.25) (layers F.Cu F.Paste F.Mask) (roundrect_rratio 0.25) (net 51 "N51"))
  (pad 6 smd roundrect (at 1.2125 1) (size 0.825 0.25) (layers F.Cu F.Paste F.Mask) (roundrect_rratio 0.25) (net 51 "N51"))
  (pad 5 smd roundrect (at -1.2125 1) (size 0.825 0.25) (layers F.Cu F.Paste F.Mask) (roundrect_rratio 0.25) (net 6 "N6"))
  (pad 4 smd roundrect (at -1.2125 0.5) (size 0.825 0.25) (layers F.Cu F.Paste F.Mask) (roundrect_rratio 0.25) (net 34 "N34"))
  (pad 3 smd roundrect (at -1.2125 0) (size 0.825 0.25) (layers F.Cu F.Paste F.Mask) (roundrect_rratio 0.25) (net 3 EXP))
  (pad 2 smd roundrect (at -1.2125 -0.5) (size 0.825 0.25) (layers F.Cu F.Paste F.Mask) (roundrect_rratio 0.25) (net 35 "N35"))
  (pad 1 smd roundrect (at -1.2125 -1) (size 0.825 0.25) (layers F.Cu F.Paste F.Mask) (roundrect_rratio 0.25) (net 2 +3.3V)))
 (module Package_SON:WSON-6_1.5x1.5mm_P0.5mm (layer F.Cu) (at 100.67 66.02 90)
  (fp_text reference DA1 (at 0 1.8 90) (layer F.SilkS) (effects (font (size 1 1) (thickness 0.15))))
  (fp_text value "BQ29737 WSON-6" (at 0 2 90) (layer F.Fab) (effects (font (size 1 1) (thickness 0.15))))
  (pad 6 smd rect (at 0.575 -0.5) (size 0.28 0.75) (layers F.Cu F.Paste F.Mask) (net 32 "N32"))
  (pad 5 smd rect (at 0.575 0) (size 0.28 0.75) (layers F.Cu F.Paste F.Mask) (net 33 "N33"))
  (pad 4 smd rect (at 0.575 0.5) (size 0.28 0.75) (layers F.Cu F.Paste F.Mask) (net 20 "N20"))
  (pad 3 smd rect (at -0.575 0.5) (size 0.28 0.75) (layers F.Cu F.Paste F.Mask) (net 28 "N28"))
  (pad 2 smd rect (at -0.575 0) (size 0.28 0.75) (layers F.Cu F.Paste F.Mask) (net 29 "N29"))
  (pad 1 smd rect (at -0.525 -0.5) (size 0.28 0.85) (layers F.Cu F.Paste F.Mask) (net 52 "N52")))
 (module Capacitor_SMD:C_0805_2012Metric (layer F.Cu) (at 98.06 53 180)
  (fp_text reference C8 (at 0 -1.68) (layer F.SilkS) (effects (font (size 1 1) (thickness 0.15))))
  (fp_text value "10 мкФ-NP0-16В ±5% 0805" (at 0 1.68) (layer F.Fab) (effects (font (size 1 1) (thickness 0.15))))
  (pad 2 smd roundrect (at 0.95 0 180) (size 1 1.45) (layers F.Cu F.Paste F.Mask) (roundrect_rratio 0.25) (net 3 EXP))
  (pad 1 smd roundrect (at -0.95 0 180) (size 1 1.45) (layers F.Cu F.Paste F.Mask) (roundrect_rratio 0.25) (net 2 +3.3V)))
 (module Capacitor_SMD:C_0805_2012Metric (layer F.Cu) (at 98.06 55.11 180)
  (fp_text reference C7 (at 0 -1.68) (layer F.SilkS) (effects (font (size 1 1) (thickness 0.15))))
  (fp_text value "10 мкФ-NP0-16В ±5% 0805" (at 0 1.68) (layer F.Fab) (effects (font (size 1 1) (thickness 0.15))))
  (pad 2 smd roundrect (at 0.95 0 180) (size 1 1.45) (layers F.Cu F.Paste F.Mask) (roundrect_rratio 0.25) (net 3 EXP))
  (pad 1 smd roundrect (at -0.95 0 180) (size 1 1.45) (layers F.Cu F.Paste F.Mask) (roundrect_rratio 0.25) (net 2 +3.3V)))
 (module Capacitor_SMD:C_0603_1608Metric (layer F.Cu) (at 96.87 94.335 270)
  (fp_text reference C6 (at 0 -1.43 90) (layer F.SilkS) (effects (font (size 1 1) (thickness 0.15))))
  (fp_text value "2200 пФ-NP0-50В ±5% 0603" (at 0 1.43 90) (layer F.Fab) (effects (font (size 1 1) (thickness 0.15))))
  (pad 2 smd roundrect (at 0.775 0 270) (size 0.9 0.95) (layers F.Cu F.Paste F.Mask) (roundrect_rratio 0.25) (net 3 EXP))
  (pad 1 smd roundrect (at -0.775 0 270) (size 0.9 0.95) (layers F.Cu F.Paste F.Mask) (roundrect_rratio 0.25) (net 1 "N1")))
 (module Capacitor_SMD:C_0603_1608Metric (layer F.Cu) (at 101.16 86.39 90)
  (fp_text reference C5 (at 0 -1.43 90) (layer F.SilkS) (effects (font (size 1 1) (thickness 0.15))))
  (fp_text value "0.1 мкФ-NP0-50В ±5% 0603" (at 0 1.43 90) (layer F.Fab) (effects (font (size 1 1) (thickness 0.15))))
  (pad 2 smd roundrect (at 0.775 0 90) (size 0.9 0.95) (layers F.Cu F.Paste F.Mask) (roundrect_rratio 0.25) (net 3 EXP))
  (pad 1 smd roundrect (at -0.775 0 90) (size 0.9 0.95) (layers F.Cu F.Paste F.Mask) (roundrect_rratio 0.25) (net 2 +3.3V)))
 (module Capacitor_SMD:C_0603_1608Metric (layer F.Cu) (at 102.98 59.48 270)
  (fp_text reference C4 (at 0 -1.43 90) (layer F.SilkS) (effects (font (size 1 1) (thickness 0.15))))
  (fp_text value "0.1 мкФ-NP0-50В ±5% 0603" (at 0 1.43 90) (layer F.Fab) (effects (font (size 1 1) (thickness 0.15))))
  (pad 2 smd roundrect (at 0.775 0 270) (size 0.9 0.95) (layers F.Cu F.Paste F.Mask) (roundrect_rratio 0.25) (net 3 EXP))
  (pad 1 smd roundrect (at -0.775 0 270) (size 0.9 0.95) (layers F.Cu F.Paste F.Mask) (roundrect_rratio 0.25) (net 51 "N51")))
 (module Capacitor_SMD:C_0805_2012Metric (layer F.Cu) (at 99.97 60.3)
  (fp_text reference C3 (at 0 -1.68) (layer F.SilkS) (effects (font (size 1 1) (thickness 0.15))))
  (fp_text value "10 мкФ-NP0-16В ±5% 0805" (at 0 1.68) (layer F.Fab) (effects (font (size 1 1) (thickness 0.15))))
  (pad 2 smd roundrect (at 0.95 0) (size 1 1.45) (layers F.Cu F.Paste F.Mask) (roundrect_rratio 0.25) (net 3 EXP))
  (pad 1 smd roundrect (at -0.95 0) (size 1 1.45) (layers F.Cu F.Paste F.Mask) (roundrect_rratio 0.25) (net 6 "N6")))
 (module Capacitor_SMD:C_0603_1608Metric (layer F.Cu) (at 102.96 63.86)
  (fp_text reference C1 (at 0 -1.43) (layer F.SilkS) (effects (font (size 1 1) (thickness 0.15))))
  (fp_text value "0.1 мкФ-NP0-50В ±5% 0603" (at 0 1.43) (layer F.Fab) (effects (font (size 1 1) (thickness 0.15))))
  (pad 2 smd roundrect (at 0.775 0) (size 0.9 0.95) (layers F.Cu F.Paste F.Mask) (roundrect_rratio 0.25) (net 20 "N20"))
  (pad 1 smd roundrect (at -0.775 0) (size 0.9 0.95) (layers F.Cu F.Paste F.Mask) (roundrect_rratio 0.25) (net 33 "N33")))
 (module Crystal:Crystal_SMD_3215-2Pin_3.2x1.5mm (layer F.Cu) (at 98.73 89.44 270)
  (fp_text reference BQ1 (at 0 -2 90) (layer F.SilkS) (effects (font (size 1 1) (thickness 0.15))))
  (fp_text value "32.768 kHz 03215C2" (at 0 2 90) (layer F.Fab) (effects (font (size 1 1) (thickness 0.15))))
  (pad 2 smd rect (at -1.25 0 270) (size 1 1.8) (layers F.Cu F.Paste F.Mask) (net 48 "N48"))
  (pad 1 smd rect (at 1.25 0 270) (size 1 1.8) (layers F.Cu F.Paste F.Mask) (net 47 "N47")))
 (gr_line (start 53 71) (end 114 71) (layer Edge.Cuts) (width 0.05))
 (gr_line (start 53 30) (end 53 71) (layer Edge.Cuts) (width 0.05))
 (gr_line (start 114 30) (end 53 30) (layer Edge.Cuts) (width 0.05))
 (gr_line (start 114 71) (end 114 30) (layer Edge.Cuts) (width 0.05))
 (segment (start 99.655 89.115) (end 98.73 88.19) (width 0.25) (layer F.Cu) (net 48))
 (segment (start 103.1075 89.115) (end 99.655 89.115) (width 0.25) (layer F.Cu) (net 48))
 (segment (start 99.655 89.765) (end 98.73 90.69) (width 0.25) (layer F.Cu) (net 47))
 (segment (start 103.1075 89.765) (end 99.655 89.765) (width 0.25) (layer F.Cu) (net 47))
 (segment (start 103.1075 87.165) (end 101.16 87.165) (width 0.25) (layer F.Cu) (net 2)))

